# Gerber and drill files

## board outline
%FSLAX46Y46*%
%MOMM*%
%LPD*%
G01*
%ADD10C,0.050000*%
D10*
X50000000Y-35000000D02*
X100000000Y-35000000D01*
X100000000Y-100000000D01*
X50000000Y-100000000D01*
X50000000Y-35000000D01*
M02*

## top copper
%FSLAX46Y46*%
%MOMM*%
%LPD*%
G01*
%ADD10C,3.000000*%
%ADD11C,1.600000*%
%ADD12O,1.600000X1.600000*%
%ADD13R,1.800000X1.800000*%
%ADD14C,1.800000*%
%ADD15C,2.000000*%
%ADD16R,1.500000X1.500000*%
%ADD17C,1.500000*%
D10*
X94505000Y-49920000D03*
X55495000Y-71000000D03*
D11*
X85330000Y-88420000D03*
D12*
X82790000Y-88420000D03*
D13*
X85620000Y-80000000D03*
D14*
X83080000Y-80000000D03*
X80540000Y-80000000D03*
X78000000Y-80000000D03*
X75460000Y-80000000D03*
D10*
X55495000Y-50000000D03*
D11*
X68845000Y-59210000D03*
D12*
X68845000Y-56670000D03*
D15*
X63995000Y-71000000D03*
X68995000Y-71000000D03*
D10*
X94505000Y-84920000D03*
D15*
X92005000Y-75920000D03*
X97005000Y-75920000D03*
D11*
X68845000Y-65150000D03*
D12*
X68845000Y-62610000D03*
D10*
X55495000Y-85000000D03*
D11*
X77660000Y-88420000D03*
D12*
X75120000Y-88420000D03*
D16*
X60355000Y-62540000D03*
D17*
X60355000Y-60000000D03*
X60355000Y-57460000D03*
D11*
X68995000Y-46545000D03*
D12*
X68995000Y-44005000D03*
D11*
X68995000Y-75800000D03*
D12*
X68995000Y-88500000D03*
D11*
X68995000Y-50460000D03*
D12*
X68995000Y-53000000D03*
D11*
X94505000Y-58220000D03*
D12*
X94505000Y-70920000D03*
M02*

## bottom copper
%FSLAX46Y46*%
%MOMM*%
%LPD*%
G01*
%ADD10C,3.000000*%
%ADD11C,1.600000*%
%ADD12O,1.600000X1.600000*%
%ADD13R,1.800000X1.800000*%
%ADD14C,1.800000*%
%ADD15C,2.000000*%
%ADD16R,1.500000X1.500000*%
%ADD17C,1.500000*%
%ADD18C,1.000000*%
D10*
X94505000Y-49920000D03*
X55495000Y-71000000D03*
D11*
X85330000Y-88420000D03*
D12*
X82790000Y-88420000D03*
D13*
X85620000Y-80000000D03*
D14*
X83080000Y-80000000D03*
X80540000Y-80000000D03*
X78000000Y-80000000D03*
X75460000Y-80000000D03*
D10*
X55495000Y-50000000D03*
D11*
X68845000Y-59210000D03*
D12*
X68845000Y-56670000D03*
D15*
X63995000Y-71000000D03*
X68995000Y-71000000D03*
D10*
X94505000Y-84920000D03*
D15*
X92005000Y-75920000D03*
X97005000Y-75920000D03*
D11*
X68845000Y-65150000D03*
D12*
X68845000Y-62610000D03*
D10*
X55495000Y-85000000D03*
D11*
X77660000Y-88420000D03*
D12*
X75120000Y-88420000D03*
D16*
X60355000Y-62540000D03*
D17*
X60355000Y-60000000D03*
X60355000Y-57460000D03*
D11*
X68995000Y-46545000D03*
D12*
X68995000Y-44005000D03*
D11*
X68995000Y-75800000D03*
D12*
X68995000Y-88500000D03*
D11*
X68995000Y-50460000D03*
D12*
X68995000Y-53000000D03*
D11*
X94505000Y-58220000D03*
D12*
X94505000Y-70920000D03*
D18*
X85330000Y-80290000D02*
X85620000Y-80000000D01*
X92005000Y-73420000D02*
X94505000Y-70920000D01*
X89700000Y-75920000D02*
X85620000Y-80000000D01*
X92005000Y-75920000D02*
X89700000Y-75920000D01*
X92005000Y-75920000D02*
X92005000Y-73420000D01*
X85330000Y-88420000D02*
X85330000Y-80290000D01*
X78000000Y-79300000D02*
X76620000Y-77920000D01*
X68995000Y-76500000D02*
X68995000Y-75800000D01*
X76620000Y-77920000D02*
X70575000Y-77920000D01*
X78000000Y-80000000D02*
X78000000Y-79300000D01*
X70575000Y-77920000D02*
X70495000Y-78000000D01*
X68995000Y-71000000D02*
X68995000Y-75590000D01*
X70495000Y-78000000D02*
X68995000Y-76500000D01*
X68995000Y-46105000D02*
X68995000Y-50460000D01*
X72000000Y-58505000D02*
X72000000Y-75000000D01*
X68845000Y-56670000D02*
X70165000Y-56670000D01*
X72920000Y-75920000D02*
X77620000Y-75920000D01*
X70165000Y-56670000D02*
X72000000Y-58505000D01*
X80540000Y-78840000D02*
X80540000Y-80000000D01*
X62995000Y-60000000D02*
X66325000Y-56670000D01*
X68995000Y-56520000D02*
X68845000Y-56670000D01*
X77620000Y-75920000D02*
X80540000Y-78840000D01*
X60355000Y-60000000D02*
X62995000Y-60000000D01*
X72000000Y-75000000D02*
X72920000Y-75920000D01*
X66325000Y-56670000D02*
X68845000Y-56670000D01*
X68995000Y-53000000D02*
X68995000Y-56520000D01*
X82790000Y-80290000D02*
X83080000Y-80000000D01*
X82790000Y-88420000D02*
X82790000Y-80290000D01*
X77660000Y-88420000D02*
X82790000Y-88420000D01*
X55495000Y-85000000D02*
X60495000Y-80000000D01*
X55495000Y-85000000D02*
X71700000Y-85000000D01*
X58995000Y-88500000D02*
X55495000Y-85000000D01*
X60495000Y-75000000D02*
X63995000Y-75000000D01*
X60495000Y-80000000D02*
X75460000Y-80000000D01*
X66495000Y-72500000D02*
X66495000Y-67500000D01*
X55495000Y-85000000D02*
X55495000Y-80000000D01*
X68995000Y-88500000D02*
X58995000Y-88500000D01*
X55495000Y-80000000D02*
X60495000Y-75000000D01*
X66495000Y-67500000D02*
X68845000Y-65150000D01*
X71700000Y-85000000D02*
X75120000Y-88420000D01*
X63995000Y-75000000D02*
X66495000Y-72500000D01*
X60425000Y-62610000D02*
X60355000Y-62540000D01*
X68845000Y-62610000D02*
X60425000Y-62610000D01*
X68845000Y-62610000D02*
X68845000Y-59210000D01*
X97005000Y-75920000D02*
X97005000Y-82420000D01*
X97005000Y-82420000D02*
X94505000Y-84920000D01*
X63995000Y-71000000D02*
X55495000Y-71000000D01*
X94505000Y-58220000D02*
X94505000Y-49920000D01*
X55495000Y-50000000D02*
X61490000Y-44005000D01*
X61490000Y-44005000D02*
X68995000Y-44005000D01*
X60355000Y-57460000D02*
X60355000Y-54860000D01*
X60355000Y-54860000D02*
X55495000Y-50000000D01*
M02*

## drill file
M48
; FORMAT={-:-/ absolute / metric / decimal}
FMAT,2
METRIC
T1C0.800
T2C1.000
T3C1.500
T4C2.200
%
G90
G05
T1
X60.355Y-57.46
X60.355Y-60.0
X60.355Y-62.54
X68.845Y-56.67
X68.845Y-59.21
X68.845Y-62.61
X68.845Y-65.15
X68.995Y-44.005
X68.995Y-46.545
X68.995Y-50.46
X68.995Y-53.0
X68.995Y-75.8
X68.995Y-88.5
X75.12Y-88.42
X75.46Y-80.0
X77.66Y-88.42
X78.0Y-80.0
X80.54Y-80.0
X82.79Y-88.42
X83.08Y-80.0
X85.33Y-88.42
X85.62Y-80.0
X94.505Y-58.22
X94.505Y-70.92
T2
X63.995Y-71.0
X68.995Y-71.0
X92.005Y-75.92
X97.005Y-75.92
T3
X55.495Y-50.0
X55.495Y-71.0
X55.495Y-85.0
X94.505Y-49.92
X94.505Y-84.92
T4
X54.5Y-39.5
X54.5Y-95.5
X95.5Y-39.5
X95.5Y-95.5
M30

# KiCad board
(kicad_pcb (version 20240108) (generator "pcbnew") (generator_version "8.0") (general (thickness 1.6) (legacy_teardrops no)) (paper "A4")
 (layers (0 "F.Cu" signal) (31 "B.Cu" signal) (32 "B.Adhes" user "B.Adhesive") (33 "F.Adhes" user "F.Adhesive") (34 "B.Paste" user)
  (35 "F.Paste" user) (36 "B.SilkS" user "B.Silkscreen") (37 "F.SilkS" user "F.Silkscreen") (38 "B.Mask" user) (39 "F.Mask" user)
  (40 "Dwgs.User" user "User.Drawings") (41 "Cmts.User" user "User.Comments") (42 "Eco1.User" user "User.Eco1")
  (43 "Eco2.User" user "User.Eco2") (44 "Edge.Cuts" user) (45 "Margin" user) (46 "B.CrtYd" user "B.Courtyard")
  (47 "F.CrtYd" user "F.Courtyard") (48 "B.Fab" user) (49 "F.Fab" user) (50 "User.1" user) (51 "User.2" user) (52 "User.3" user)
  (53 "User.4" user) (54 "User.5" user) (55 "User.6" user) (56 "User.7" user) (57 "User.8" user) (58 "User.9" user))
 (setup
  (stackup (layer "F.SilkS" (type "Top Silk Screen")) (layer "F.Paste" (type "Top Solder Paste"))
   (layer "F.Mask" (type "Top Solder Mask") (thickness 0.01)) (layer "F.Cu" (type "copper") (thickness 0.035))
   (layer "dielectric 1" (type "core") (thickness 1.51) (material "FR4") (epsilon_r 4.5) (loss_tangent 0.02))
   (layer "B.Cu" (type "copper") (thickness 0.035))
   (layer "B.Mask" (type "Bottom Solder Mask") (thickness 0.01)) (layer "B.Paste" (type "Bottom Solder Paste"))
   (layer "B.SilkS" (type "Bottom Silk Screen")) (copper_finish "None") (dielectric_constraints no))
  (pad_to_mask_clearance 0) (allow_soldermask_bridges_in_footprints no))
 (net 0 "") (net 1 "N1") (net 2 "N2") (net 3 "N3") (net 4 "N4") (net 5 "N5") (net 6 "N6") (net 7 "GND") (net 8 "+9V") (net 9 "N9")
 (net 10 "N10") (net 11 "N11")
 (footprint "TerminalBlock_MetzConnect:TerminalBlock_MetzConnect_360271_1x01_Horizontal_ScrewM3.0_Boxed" (layer "F.Cu") (at 94.505 49.92 90)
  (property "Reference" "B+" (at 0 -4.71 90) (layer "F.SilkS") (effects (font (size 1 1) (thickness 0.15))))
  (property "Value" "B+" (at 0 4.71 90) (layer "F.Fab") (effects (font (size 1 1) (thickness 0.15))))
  (pad "1" thru_hole circle (at 0 0 90) (size 3 3) (drill 1.5) (layers "*.Cu" "*.Mask") (remove_unused_layers no) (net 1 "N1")))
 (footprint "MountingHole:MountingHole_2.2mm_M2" (layer "F.Cu") (at 54.5 95.5)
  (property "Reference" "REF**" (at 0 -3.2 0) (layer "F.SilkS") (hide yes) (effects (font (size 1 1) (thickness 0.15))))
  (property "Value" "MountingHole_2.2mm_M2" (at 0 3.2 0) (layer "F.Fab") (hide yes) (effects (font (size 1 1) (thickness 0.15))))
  (pad "" np_thru_hole circle (at 0 0) (size 2.2 2.2) (drill 2.2) (layers "*.Cu" "*.Mask")))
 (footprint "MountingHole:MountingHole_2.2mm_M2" (layer "F.Cu") (at 95.5 39.5)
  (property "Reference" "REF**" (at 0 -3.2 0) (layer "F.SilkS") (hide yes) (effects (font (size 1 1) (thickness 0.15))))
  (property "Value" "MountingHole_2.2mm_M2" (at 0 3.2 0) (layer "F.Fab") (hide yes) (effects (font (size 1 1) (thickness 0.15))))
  (pad "" np_thru_hole circle (at 0 0) (size 2.2 2.2) (drill 2.2) (layers "*.Cu" "*.Mask")))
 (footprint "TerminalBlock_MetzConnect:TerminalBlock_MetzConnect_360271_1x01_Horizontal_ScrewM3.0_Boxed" (layer "F.Cu") (at 55.495 71 -90)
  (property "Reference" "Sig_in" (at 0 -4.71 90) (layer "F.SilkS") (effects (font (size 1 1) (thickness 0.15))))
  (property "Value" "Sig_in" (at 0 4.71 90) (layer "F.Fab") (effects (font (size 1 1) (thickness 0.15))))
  (pad "1" thru_hole circle (at 0 0 270) (size 3 3) (drill 1.5) (layers "*.Cu" "*.Mask") (remove_unused_layers no) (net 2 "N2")))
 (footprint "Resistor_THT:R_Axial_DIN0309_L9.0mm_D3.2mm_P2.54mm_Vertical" (layer "F.Cu") (at 85.33 88.42 180)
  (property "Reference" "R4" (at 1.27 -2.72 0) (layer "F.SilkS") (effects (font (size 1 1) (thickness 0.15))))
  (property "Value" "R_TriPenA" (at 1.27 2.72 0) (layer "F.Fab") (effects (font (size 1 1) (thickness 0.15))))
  (pad "1" thru_hole circle (at 0 0 180) (size 1.6 1.6) (drill 0.8) (layers "*.Cu" "*.Mask") (remove_unused_layers no) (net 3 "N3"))
  (pad "2" thru_hole oval (at 2.54 0 180) (size 1.6 1.6) (drill 0.8) (layers "*.Cu" "*.Mask") (remove_unused_layers no) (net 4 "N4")))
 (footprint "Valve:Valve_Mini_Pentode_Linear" (layer "F.Cu") (at 85.62 80 180)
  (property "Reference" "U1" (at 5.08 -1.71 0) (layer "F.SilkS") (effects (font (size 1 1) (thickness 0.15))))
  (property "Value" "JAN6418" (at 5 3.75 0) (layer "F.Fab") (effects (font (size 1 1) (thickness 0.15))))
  (pad "1" thru_hole rect (at 0 0 180) (size 1.8 1.8) (drill 0.8) (layers "*.Cu" "*.Mask") (remove_unused_layers no) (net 3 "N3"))
  (pad "2" thru_hole circle (at 2.54 0 180) (size 1.8 1.8) (drill 0.8) (layers "*.Cu" "*.Mask") (remove_unused_layers no) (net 4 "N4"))
  (pad "3" thru_hole circle (at 5.08 0 180) (size 1.8 1.8) (drill 0.8) (layers "*.Cu" "*.Mask") (remove_unused_layers no) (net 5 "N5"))
  (pad "4" thru_hole circle (at 7.62 0 180) (size 1.8 1.8) (drill 0.8) (layers "*.Cu" "*.Mask") (remove_unused_layers no) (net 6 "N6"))
  (pad "5" thru_hole circle (at 10.16 0 180) (size 1.8 1.8) (drill 0.8) (layers "*.Cu" "*.Mask") (remove_unused_layers no) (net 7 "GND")))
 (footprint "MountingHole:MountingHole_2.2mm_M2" (layer "F.Cu") (at 95.5 95.5)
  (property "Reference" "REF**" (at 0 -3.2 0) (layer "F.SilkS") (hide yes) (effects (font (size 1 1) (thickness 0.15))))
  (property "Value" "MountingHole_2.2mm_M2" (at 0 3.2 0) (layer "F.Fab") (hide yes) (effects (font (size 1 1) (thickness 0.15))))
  (pad "" np_thru_hole circle (at 0 0) (size 2.2 2.2) (drill 2.2) (layers "*.Cu" "*.Mask")))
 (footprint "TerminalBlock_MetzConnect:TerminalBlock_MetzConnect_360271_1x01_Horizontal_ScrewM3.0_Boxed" (layer "F.Cu") (at 55.495 50 -90)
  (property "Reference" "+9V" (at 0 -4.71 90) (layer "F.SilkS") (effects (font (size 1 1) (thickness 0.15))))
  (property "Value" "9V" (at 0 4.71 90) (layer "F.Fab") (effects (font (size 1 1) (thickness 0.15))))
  (pad "1" thru_hole circle (at 0 0 270) (size 3 3) (drill 1.5) (layers "*.Cu" "*.Mask") (remove_unused_layers no) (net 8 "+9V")))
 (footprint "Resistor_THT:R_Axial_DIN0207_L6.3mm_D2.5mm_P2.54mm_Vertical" (layer "F.Cu") (at 68.845 59.21 90)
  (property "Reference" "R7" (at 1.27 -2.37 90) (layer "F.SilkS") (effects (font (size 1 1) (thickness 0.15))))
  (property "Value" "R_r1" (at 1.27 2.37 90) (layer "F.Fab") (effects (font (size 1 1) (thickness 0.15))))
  (pad "1" thru_hole circle (at 0 0 90) (size 1.6 1.6) (drill 0.8) (layers "*.Cu" "*.Mask") (remove_unused_layers no) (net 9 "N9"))
  (pad "2" thru_hole oval (at 2.54 0 90) (size 1.6 1.6) (drill 0.8) (layers "*.Cu" "*.Mask") (remove_unused_layers no) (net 5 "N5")))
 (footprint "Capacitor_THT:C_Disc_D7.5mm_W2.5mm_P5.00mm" (layer "F.Cu") (at 63.995 71)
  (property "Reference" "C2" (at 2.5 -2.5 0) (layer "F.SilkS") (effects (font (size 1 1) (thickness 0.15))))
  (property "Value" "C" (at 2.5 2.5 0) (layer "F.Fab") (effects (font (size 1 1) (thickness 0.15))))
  (pad "1" thru_hole circle (at 0 0) (size 2 2) (drill 1) (layers "*.Cu" "*.Mask") (remove_unused_layers no) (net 2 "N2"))
  (pad "2" thru_hole circle (at 5 0) (size 2 2) (drill 1) (layers "*.Cu" "*.Mask") (remove_unused_layers no) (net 6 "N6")))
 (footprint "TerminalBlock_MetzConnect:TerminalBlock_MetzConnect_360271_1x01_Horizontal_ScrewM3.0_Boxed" (layer "F.Cu") (at 94.505 84.92 90)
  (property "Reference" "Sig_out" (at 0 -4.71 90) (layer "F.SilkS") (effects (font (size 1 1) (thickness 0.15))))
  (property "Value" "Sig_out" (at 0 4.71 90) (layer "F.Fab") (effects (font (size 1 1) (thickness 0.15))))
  (pad "1" thru_hole circle (at 0 0 90) (size 3 3) (drill 1.5) (layers "*.Cu" "*.Mask") (remove_unused_layers no) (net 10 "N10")))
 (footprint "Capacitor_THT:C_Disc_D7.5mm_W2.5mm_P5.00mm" (layer "F.Cu") (at 92.005 75.92)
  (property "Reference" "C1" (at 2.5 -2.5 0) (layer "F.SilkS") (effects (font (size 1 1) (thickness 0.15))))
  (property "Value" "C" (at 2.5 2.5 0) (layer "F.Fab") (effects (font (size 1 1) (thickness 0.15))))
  (pad "1" thru_hole circle (at 0 0) (size 2 2) (drill 1) (layers "*.Cu" "*.Mask") (remove_unused_layers no) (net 3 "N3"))
  (pad "2" thru_hole circle (at 5 0) (size 2 2) (drill 1) (layers "*.Cu" "*.Mask") (remove_unused_layers no) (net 10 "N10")))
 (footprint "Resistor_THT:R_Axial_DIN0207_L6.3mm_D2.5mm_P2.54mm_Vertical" (layer "F.Cu") (at 68.845 65.15 90)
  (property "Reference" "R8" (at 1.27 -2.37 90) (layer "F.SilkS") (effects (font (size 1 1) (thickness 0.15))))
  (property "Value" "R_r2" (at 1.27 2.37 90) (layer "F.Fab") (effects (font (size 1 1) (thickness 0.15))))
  (pad "1" thru_hole circle (at 0 0 90) (size 1.6 1.6) (drill 0.8) (layers "*.Cu" "*.Mask") (remove_unused_layers no) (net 7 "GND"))
  (pad "2" thru_hole oval (at 2.54 0 90) (size 1.6 1.6) (drill 0.8) (layers "*.Cu" "*.Mask") (remove_unused_layers no) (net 9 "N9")))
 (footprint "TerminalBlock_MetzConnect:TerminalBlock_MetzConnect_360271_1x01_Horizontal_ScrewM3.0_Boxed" (layer "F.Cu") (at 55.495 85 -90)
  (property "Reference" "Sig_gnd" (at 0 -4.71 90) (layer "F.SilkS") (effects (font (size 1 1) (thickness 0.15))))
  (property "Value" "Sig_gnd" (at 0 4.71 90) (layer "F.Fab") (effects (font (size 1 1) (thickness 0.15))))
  (pad "1" thru_hole circle (at 0 0 270) (size 3 3) (drill 1.5) (layers "*.Cu" "*.Mask") (remove_unused_layers no) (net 7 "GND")))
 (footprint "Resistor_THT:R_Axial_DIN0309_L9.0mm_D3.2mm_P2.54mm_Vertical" (layer "F.Cu") (at 77.66 88.42 180)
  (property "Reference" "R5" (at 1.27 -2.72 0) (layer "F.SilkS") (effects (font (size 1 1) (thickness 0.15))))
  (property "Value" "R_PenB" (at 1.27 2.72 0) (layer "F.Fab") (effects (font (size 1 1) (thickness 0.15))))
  (pad "1" thru_hole circle (at 0 0 180) (size 1.6 1.6) (drill 0.8) (layers "*.Cu" "*.Mask") (remove_unused_layers no) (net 4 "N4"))
  (pad "2" thru_hole oval (at 2.54 0 180) (size 1.6 1.6) (drill 0.8) (layers "*.Cu" "*.Mask") (remove_unused_layers no) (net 7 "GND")))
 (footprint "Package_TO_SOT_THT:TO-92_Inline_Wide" (layer "F.Cu") (at 60.355 62.54 90)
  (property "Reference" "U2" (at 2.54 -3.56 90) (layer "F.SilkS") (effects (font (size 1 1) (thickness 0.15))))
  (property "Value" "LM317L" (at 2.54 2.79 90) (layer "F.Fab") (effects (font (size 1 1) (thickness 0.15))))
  (pad "1" thru_hole rect (at 0 0 90) (size 1.5 1.5) (drill 0.8) (layers "*.Cu" "*.Mask") (remove_unused_layers no) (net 9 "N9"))
  (pad "2" thru_hole circle (at 2.54 0 90) (size 1.5 1.5) (drill 0.8) (layers "*.Cu" "*.Mask") (remove_unused_layers no) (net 5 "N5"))
  (pad "3" thru_hole circle (at 5.08 0 90) (size 1.5 1.5) (drill 0.8) (layers "*.Cu" "*.Mask") (remove_unused_layers no) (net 8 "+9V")))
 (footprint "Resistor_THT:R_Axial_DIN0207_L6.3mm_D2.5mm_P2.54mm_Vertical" (layer "F.Cu") (at 68.995 46.545 90)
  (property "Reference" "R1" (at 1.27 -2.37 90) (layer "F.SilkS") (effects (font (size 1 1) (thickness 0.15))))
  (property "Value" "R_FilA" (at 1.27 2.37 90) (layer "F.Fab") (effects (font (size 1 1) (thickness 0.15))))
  (pad "1" thru_hole circle (at 0 0 90) (size 1.6 1.6) (drill 0.8) (layers "*.Cu" "*.Mask") (remove_unused_layers no) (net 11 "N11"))
  (pad "2" thru_hole oval (at 2.54 0 90) (size 1.6 1.6) (drill 0.8) (layers "*.Cu" "*.Mask") (remove_unused_layers no) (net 8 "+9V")))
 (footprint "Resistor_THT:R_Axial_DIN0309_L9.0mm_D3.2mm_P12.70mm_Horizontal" (layer "F.Cu") (at 68.995 75.8 -90)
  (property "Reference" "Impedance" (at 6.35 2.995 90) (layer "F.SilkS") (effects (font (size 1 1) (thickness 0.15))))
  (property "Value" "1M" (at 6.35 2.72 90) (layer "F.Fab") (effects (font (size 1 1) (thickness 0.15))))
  (pad "1" thru_hole circle (at 0 0 270) (size 1.6 1.6) (drill 0.8) (layers "*.Cu" "*.Mask") (remove_unused_layers no) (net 6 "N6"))
  (pad "2" thru_hole oval (at 12.7 0 270) (size 1.6 1.6) (drill 0.8) (layers "*.Cu" "*.Mask") (remove_unused_layers no) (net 7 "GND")))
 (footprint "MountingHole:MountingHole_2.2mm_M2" (layer "F.Cu") (at 54.5 39.5)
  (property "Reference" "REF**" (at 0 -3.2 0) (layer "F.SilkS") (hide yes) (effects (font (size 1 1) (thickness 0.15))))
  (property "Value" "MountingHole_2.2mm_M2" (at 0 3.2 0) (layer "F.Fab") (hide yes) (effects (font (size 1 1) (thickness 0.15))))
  (pad "" np_thru_hole circle (at 0 0) (size 2.2 2.2) (drill 2.2) (layers "*.Cu" "*.Mask")))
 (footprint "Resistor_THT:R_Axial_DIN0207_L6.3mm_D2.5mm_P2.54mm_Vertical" (layer "F.Cu") (at 68.995 50.46 -90)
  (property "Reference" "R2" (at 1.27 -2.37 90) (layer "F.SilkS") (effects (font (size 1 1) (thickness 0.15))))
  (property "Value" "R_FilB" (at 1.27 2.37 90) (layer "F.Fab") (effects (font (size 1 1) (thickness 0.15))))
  (pad "1" thru_hole circle (at 0 0 270) (size 1.6 1.6) (drill 0.8) (layers "*.Cu" "*.Mask") (remove_unused_layers no) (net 11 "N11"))
  (pad "2" thru_hole oval (at 2.54 0 270) (size 1.6 1.6) (drill 0.8) (layers "*.Cu" "*.Mask") (remove_unused_layers no) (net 5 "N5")))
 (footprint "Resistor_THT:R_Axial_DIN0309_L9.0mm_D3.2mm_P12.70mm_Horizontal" (layer "F.Cu") (at 94.505 58.22 -90)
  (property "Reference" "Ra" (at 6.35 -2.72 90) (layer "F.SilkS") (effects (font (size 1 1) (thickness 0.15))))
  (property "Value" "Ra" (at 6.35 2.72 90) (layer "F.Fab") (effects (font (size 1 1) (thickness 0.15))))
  (pad "1" thru_hole circle (at 0 0 270) (size 1.6 1.6) (drill 0.8) (layers "*.Cu" "*.Mask") (remove_unused_layers no) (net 1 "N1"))
  (pad "2" thru_hole oval (at 12.7 0 270) (size 1.6 1.6) (drill 0.8) (layers "*.Cu" "*.Mask") (remove_unused_layers no) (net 3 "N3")))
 (gr_rect (start 50 35) (end 100 100) (stroke (width 0.05) (type default)) (fill none) (layer "Edge.Cuts"))
 (segment (start 85.33 80.29) (end 85.62 80) (width 1) (layer "B.Cu") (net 3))
 (segment (start 92.005 73.42) (end 94.505 70.92) (width 1) (layer "B.Cu") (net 3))
 (segment (start 89.7 75.92) (end 85.62 80) (width 1) (layer "B.Cu") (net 3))
 (segment (start 92.005 75.92) (end 89.7 75.92) (width 1) (layer "B.Cu") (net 3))
 (segment (start 92.005 75.92) (end 92.005 73.42) (width 1) (layer "B.Cu") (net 3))
 (segment (start 85.33 88.42) (end 85.33 80.29) (width 1) (layer "B.Cu") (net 3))
 (segment (start 78 79.3) (end 76.62 77.92) (width 1) (layer "B.Cu") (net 6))
 (segment (start 68.995 76.5) (end 68.995 75.8) (width 1) (layer "B.Cu") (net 6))
 (segment (start 76.62 77.92) (end 70.575 77.92) (width 1) (layer "B.Cu") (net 6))
 (segment (start 78 80) (end 78 79.3) (width 1) (layer "B.Cu") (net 6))
 (segment (start 70.575 77.92) (end 70.495 78) (width 1) (layer "B.Cu") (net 6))
 (segment (start 68.995 71) (end 68.995 75.59) (width 1) (layer "B.Cu") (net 6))
 (segment (start 70.495 78) (end 68.995 76.5) (width 1) (layer "B.Cu") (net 6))
 (segment (start 68.995 46.105) (end 68.995 50.46) (width 1) (layer "B.Cu") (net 11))
 (segment (start 72 58.505) (end 72 75) (width 1) (layer "B.Cu") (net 5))
 (segment (start 68.845 56.67) (end 70.165 56.67) (width 1) (layer "B.Cu") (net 5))
 (segment (start 72.92 75.92) (end 77.62 75.92) (width 1) (layer "B.Cu") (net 5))
 (segment (start 70.165 56.67) (end 72 58.505) (width 1) (layer "B.Cu") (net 5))
 (segment (start 80.54 78.84) (end 80.54 80) (width 1) (layer "B.Cu") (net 5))
 (segment (start 62.995 60) (end 66.325 56.67) (width 1) (layer "B.Cu") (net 5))
 (segment (start 68.995 56.52) (end 68.845 56.67) (width 1) (layer "B.Cu") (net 5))
 (segment (start 77.62 75.92) (end 80.54 78.84) (width 1) (layer "B.Cu") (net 5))
 (segment (start 60.355 60) (end 62.995 60) (width 1) (layer "B.Cu") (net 5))
 (segment (start 72 75) (end 72.92 75.92) (width 1) (layer "B.Cu") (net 5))
 (segment (start 66.325 56.67) (end 68.845 56.67) (width 1) (layer "B.Cu") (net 5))
 (segment (start 68.995 53) (end 68.995 56.52) (width 1) (layer "B.Cu") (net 5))
 (segment (start 82.79 80.29) (end 83.08 80) (width 1) (layer "B.Cu") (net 4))
 (segment (start 82.79 88.42) (end 82.79 80.29) (width 1) (layer "B.Cu") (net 4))
 (segment (start 77.66 88.42) (end 82.79 88.42) (width 1) (layer "B.Cu") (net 4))
 (segment (start 55.495 85) (end 60.495 80) (width 1) (layer "B.Cu") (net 7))
 (segment (start 55.495 85) (end 71.7 85) (width 1) (layer "B.Cu") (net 7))
 (segment (start 58.995 88.5) (end 55.495 85) (width 1) (layer "B.Cu") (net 7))
 (segment (start 60.495 75) (end 63.995 75) (width 1) (layer "B.Cu") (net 7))
 (segment (start 60.495 80) (end 75.46 80) (width 1) (layer "B.Cu") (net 7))
 (segment (start 66.495 72.5) (end 66.495 67.5) (width 1) (layer "B.Cu") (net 7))
 (segment (start 55.495 85) (end 55.495 80) (width 1) (layer "B.Cu") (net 7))
 (segment (start 68.995 88.5) (end 58.995 88.5) (width 1) (layer "B.Cu") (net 7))
 (segment (start 55.495 80) (end 60.495 75) (width 1) (layer "B.Cu") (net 7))
 (segment (start 66.495 67.5) (end 68.845 65.15) (width 1) (layer "B.Cu") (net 7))
 (segment (start 71.7 85) (end 75.12 88.42) (width 1) (layer "B.Cu") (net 7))
 (segment (start 63.995 75) (end 66.495 72.5) (width 1) (layer "B.Cu") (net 7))
 (segment (start 60.425 62.61) (end 60.355 62.54) (width 1) (layer "B.Cu") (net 9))
 (segment (start 68.845 62.61) (end 60.425 62.61) (width 1) (layer "B.Cu") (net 9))
 (segment (start 68.845 62.61) (end 68.845 59.21) (width 1) (layer "B.Cu") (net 9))
 (segment (start 97.005 75.92) (end 97.005 82.42) (width 1) (layer "B.Cu") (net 10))
 (segment (start 97.005 82.42) (end 94.505 84.92) (width 1) (layer "B.Cu") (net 10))
 (segment (start 63.995 71) (end 55.495 71) (width 1) (layer "B.Cu") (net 2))
 (segment (start 94.505 58.22) (end 94.505 49.92) (width 1) (layer "B.Cu") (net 1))
 (segment (start 55.495 50) (end 61.49 44.005) (width 1) (layer "B.Cu") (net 8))
 (segment (start 61.49 44.005) (end 68.995 44.005) (width 1) (layer "B.Cu") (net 8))
 (segment (start 60.355 57.46) (end 60.355 54.86) (width 1) (layer "B.Cu") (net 8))
 (segment (start 60.355 54.86) (end 55.495 50) (width 1) (layer "B.Cu") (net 8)))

